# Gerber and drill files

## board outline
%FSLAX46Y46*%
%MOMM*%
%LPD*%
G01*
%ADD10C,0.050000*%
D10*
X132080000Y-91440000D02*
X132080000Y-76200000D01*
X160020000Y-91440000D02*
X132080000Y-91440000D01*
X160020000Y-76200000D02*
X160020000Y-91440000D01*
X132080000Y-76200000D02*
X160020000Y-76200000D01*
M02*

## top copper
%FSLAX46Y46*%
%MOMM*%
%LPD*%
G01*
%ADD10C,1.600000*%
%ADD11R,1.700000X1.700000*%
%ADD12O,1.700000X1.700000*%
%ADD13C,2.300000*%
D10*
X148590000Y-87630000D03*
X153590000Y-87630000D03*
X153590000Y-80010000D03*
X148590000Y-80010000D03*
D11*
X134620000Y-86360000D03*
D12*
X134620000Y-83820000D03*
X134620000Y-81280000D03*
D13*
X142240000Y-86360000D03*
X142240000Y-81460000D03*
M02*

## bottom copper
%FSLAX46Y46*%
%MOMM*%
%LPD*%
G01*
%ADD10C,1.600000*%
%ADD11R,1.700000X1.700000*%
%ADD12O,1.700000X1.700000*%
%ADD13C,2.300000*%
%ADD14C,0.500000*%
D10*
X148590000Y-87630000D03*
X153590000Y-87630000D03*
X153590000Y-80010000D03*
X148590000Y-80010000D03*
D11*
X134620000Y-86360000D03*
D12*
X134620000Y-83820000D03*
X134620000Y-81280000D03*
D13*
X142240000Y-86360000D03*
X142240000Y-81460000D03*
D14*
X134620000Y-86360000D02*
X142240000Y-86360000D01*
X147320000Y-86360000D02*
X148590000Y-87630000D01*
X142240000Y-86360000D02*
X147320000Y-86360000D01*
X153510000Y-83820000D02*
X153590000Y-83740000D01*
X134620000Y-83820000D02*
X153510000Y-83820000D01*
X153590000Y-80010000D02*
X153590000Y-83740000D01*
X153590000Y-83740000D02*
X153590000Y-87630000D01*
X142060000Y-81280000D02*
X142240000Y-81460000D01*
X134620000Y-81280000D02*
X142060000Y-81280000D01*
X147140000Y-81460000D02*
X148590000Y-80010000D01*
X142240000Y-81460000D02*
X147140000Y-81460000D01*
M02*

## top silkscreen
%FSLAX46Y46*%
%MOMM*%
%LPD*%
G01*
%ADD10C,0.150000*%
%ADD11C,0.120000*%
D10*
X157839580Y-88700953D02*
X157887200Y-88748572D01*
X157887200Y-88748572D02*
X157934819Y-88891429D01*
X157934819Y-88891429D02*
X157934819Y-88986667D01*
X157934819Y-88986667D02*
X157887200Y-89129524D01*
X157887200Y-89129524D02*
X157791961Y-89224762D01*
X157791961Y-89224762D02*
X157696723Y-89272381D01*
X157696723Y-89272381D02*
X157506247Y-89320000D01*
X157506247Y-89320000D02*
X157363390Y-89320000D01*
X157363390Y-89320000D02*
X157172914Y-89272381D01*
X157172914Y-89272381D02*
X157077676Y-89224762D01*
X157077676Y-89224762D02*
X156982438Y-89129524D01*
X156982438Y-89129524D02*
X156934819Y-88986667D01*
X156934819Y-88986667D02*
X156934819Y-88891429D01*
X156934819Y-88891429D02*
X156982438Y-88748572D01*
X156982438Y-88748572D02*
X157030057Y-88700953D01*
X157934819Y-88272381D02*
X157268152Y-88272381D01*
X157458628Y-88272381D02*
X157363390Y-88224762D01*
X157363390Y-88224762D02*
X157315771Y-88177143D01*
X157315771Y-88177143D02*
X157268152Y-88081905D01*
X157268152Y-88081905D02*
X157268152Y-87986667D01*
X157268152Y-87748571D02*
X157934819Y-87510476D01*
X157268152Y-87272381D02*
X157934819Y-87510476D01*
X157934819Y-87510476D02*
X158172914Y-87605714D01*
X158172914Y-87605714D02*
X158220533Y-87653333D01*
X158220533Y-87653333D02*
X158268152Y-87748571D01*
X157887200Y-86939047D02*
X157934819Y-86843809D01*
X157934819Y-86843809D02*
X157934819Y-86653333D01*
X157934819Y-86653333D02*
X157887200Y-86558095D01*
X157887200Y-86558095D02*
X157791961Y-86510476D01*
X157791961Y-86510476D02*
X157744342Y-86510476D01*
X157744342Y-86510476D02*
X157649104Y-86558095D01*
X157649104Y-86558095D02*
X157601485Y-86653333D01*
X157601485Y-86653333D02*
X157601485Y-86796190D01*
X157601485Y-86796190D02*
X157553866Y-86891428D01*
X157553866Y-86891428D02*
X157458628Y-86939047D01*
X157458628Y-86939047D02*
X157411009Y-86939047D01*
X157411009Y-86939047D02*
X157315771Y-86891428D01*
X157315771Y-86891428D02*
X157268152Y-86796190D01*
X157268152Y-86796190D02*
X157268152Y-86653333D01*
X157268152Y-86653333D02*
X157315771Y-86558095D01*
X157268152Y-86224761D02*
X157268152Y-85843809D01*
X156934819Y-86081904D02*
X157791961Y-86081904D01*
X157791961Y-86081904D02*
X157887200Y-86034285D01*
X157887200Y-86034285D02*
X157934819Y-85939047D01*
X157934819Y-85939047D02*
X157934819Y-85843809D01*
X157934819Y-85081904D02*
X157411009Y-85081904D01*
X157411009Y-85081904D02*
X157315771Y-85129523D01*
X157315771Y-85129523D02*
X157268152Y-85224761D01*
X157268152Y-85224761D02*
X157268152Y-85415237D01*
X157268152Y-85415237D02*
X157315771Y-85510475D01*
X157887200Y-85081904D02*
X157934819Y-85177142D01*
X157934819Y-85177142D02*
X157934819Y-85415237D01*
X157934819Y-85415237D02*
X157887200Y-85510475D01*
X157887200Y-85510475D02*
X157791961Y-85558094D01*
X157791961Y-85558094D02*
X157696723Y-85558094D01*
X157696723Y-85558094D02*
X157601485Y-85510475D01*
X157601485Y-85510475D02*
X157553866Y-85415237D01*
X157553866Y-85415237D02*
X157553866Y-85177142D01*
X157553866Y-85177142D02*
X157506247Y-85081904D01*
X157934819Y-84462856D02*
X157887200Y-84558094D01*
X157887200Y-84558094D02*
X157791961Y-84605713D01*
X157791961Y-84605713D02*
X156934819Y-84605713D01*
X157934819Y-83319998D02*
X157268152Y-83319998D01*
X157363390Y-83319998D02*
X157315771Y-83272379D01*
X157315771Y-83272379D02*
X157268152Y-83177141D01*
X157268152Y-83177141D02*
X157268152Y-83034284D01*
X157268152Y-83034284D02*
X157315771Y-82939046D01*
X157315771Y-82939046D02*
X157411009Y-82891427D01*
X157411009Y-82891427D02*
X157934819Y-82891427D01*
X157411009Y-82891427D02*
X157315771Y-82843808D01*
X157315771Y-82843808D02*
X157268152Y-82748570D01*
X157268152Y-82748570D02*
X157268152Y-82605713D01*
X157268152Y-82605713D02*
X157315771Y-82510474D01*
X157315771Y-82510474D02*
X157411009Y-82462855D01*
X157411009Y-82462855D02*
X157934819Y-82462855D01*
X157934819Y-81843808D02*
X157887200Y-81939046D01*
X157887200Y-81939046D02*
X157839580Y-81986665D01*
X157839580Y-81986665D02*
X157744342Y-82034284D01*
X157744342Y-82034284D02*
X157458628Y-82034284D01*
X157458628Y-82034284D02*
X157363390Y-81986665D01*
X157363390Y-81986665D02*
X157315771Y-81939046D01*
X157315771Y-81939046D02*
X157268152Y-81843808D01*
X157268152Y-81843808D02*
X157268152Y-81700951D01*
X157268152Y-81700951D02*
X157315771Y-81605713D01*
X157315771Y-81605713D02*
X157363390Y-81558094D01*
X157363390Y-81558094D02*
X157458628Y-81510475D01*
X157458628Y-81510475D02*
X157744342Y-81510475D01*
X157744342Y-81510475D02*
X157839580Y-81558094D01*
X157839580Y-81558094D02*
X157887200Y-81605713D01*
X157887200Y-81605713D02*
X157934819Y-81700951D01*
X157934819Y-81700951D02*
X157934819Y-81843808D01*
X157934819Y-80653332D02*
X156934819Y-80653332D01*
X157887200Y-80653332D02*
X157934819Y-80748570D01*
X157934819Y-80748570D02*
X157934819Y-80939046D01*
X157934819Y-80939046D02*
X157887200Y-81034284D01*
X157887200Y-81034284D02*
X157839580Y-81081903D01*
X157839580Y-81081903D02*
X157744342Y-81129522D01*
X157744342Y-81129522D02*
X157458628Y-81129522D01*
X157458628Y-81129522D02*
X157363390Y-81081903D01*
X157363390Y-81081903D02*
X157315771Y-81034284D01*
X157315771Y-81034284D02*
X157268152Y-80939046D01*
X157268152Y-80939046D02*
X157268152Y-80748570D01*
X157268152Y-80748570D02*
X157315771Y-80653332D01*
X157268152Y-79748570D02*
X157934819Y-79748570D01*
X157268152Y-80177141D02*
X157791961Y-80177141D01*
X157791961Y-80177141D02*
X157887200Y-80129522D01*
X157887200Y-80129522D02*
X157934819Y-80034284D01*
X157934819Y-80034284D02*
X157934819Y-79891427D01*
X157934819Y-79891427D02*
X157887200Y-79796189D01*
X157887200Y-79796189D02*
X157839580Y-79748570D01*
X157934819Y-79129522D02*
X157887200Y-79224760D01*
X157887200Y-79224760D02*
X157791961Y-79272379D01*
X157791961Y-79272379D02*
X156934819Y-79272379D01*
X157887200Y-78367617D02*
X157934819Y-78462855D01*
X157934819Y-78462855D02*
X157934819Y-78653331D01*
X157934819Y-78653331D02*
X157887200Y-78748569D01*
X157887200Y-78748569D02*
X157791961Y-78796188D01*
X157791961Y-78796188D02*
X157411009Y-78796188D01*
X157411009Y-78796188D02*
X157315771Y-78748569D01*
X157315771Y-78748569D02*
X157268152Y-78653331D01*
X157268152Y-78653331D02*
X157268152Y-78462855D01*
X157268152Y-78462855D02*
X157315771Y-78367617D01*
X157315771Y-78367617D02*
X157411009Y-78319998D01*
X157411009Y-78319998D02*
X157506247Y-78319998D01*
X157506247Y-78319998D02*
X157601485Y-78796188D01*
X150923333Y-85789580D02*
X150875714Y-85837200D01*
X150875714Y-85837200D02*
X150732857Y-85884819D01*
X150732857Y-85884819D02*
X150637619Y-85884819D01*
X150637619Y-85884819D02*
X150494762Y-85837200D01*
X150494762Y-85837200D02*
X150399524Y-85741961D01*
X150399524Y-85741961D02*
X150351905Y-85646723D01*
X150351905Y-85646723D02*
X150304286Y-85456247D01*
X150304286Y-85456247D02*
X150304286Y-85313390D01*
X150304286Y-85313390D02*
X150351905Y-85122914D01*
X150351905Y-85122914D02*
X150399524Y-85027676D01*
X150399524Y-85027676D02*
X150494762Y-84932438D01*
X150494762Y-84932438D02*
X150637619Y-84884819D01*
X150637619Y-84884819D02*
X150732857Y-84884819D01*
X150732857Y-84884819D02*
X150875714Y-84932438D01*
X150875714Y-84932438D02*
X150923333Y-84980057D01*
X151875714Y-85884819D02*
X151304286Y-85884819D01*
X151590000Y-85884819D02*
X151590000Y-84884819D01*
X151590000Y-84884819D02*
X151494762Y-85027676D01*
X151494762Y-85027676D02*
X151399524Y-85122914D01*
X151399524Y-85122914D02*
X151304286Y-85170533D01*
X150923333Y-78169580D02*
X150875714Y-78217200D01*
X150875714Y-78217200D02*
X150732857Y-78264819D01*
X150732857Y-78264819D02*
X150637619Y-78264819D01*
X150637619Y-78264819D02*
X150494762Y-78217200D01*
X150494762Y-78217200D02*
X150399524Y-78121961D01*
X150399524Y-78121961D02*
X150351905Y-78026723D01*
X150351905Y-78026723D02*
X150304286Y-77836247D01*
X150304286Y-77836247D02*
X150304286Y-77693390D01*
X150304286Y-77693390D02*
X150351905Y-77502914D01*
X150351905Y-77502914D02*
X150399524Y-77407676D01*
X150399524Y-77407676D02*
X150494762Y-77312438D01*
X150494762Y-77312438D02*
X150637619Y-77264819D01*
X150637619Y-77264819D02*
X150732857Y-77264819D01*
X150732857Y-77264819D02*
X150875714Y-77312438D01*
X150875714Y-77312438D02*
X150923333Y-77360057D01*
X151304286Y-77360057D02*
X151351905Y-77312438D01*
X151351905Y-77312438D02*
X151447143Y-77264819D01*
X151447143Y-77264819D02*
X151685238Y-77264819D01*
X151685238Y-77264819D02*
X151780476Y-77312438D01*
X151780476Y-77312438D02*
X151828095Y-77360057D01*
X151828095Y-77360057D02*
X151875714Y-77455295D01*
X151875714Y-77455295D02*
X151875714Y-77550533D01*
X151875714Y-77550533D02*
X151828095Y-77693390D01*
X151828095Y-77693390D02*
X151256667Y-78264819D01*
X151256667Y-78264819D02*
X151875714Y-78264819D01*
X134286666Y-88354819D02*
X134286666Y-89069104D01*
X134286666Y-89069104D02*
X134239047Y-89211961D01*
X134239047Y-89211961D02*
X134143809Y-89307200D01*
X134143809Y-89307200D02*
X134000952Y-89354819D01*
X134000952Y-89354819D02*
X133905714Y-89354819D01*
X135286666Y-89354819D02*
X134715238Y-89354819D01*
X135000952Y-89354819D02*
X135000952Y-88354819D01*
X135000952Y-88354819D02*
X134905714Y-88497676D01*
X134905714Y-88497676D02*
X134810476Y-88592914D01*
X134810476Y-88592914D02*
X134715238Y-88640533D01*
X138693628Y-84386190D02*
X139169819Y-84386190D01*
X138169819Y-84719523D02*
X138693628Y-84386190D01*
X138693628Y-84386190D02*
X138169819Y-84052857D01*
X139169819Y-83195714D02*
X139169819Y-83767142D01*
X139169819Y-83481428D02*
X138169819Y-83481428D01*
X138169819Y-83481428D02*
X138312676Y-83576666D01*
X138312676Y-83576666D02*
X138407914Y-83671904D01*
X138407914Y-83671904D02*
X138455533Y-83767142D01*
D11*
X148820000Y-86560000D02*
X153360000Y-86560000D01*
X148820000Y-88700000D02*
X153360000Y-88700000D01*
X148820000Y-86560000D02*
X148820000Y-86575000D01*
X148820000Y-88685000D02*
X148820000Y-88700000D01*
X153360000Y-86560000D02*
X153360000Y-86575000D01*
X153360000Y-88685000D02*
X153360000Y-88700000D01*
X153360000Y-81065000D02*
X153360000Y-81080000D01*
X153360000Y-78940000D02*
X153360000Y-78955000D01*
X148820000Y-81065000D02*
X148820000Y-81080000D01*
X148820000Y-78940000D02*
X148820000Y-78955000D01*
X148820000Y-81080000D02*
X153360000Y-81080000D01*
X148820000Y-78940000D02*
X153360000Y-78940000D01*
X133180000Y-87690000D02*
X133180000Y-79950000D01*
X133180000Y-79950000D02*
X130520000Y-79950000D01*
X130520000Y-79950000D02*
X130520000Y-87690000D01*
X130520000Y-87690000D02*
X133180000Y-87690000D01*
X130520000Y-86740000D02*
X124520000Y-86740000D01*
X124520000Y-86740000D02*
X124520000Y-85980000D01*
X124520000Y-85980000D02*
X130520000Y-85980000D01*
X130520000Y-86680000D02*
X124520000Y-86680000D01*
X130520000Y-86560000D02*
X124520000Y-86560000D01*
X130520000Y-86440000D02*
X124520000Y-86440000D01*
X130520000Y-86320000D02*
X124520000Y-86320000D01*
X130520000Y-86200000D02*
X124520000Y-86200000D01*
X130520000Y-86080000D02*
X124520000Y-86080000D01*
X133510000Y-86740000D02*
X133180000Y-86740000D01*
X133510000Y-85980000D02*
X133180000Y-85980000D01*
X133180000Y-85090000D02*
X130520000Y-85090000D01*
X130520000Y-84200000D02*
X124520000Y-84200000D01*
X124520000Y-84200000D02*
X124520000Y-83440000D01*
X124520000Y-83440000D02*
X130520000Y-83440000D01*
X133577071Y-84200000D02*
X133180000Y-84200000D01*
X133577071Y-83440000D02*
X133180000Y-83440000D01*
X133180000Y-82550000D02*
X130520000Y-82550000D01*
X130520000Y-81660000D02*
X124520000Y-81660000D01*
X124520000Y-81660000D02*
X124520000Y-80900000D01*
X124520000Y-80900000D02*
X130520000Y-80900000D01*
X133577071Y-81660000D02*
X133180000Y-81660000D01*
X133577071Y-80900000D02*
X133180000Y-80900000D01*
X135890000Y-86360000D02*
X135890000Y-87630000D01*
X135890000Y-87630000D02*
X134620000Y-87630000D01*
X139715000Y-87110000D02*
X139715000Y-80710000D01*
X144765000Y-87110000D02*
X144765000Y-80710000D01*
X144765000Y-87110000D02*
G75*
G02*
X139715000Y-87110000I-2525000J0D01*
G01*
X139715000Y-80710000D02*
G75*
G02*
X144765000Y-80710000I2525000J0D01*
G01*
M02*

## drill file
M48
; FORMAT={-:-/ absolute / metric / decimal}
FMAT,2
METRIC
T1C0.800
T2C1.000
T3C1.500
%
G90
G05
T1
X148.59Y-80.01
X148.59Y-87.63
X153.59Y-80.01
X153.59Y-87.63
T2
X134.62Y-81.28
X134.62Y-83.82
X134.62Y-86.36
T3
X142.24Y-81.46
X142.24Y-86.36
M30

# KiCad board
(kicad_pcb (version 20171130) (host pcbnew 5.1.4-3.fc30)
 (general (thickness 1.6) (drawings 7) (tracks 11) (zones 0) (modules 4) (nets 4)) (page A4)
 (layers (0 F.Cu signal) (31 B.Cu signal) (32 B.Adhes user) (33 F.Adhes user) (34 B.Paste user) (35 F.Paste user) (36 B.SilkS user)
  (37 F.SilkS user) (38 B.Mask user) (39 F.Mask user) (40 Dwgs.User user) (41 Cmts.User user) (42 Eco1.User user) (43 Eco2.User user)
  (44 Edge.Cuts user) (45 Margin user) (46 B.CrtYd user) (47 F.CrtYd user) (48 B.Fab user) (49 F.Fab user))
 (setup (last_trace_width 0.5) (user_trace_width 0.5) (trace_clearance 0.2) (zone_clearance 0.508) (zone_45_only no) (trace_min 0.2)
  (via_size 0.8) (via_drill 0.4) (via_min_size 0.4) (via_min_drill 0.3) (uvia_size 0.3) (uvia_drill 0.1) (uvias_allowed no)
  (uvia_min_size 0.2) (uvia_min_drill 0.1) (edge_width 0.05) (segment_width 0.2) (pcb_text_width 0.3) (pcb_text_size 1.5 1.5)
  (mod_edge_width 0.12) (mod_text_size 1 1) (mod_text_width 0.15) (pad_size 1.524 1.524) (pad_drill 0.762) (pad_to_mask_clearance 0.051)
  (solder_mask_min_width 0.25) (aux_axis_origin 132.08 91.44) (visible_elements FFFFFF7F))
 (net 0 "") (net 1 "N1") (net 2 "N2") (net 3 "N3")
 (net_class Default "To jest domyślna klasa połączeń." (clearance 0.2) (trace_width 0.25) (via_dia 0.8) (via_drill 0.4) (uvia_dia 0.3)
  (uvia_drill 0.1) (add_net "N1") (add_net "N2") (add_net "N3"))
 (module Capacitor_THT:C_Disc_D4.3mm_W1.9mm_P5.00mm (layer F.Cu) (at 148.59 87.63)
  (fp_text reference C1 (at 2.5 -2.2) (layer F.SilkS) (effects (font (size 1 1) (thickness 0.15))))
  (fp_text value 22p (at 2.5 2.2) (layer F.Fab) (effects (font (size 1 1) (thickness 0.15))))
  (fp_line (start 0.23 -1.07) (end 4.77 -1.07) (layer F.SilkS) (width 0.12))
  (fp_line (start 0.23 1.07) (end 4.77 1.07) (layer F.SilkS) (width 0.12))
  (fp_line (start 0.23 -1.07) (end 0.23 -1.055) (layer F.SilkS) (width 0.12))
  (fp_line (start 0.23 1.055) (end 0.23 1.07) (layer F.SilkS) (width 0.12))
  (fp_line (start 4.77 -1.07) (end 4.77 -1.055) (layer F.SilkS) (width 0.12))
  (fp_line (start 4.77 1.055) (end 4.77 1.07) (layer F.SilkS) (width 0.12))
  (pad 1 thru_hole circle (at 0 0) (size 1.6 1.6) (drill 0.8) (layers *.Cu *.Mask) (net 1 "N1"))
  (pad 2 thru_hole circle (at 5 0) (size 1.6 1.6) (drill 0.8) (layers *.Cu *.Mask) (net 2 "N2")))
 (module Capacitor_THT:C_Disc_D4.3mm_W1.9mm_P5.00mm (layer F.Cu) (at 148.59 80.01)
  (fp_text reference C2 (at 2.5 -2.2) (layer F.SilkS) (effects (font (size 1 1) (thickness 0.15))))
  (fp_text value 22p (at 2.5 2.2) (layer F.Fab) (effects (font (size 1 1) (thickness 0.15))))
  (fp_line (start 4.77 1.055) (end 4.77 1.07) (layer F.SilkS) (width 0.12))
  (fp_line (start 4.77 -1.07) (end 4.77 -1.055) (layer F.SilkS) (width 0.12))
  (fp_line (start 0.23 1.055) (end 0.23 1.07) (layer F.SilkS) (width 0.12))
  (fp_line (start 0.23 -1.07) (end 0.23 -1.055) (layer F.SilkS) (width 0.12))
  (fp_line (start 0.23 1.07) (end 4.77 1.07) (layer F.SilkS) (width 0.12))
  (fp_line (start 0.23 -1.07) (end 4.77 -1.07) (layer F.SilkS) (width 0.12))
  (pad 2 thru_hole circle (at 5 0) (size 1.6 1.6) (drill 0.8) (layers *.Cu *.Mask) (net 2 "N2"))
  (pad 1 thru_hole circle (at 0 0) (size 1.6 1.6) (drill 0.8) (layers *.Cu *.Mask) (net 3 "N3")))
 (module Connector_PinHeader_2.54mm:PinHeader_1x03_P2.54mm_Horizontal (layer F.Cu) (at 134.62 86.36 180)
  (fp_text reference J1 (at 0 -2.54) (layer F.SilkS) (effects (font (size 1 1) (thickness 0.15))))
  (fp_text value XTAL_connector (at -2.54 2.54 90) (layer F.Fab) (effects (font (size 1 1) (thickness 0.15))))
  (fp_line (start 1.44 -1.33) (end 1.44 6.41) (layer F.SilkS) (width 0.12))
  (fp_line (start 1.44 6.41) (end 4.1 6.41) (layer F.SilkS) (width 0.12))
  (fp_line (start 4.1 6.41) (end 4.1 -1.33) (layer F.SilkS) (width 0.12))
  (fp_line (start 4.1 -1.33) (end 1.44 -1.33) (layer F.SilkS) (width 0.12))
  (fp_line (start 4.1 -0.38) (end 10.1 -0.38) (layer F.SilkS) (width 0.12))
  (fp_line (start 10.1 -0.38) (end 10.1 0.38) (layer F.SilkS) (width 0.12))
  (fp_line (start 10.1 0.38) (end 4.1 0.38) (layer F.SilkS) (width 0.12))
  (fp_line (start 4.1 -0.32) (end 10.1 -0.32) (layer F.SilkS) (width 0.12))
  (fp_line (start 4.1 -0.2) (end 10.1 -0.2) (layer F.SilkS) (width 0.12))
  (fp_line (start 4.1 -0.08) (end 10.1 -0.08) (layer F.SilkS) (width 0.12))
  (fp_line (start 4.1 0.04) (end 10.1 0.04) (layer F.SilkS) (width 0.12))
  (fp_line (start 4.1 0.16) (end 10.1 0.16) (layer F.SilkS) (width 0.12))
  (fp_line (start 4.1 0.28) (end 10.1 0.28) (layer F.SilkS) (width 0.12))
  (fp_line (start 1.11 -0.38) (end 1.44 -0.38) (layer F.SilkS) (width 0.12))
  (fp_line (start 1.11 0.38) (end 1.44 0.38) (layer F.SilkS) (width 0.12))
  (fp_line (start 1.44 1.27) (end 4.1 1.27) (layer F.SilkS) (width 0.12))
  (fp_line (start 4.1 2.16) (end 10.1 2.16) (layer F.SilkS) (width 0.12))
  (fp_line (start 10.1 2.16) (end 10.1 2.92) (layer F.SilkS) (width 0.12))
  (fp_line (start 10.1 2.92) (end 4.1 2.92) (layer F.SilkS) (width 0.12))
  (fp_line (start 1.042929 2.16) (end 1.44 2.16) (layer F.SilkS) (width 0.12))
  (fp_line (start 1.042929 2.92) (end 1.44 2.92) (layer F.SilkS) (width 0.12))
  (fp_line (start 1.44 3.81) (end 4.1 3.81) (layer F.SilkS) (width 0.12))
  (fp_line (start 4.1 4.7) (end 10.1 4.7) (layer F.SilkS) (width 0.12))
  (fp_line (start 10.1 4.7) (end 10.1 5.46) (layer F.SilkS) (width 0.12))
  (fp_line (start 10.1 5.46) (end 4.1 5.46) (layer F.SilkS) (width 0.12))
  (fp_line (start 1.042929 4.7) (end 1.44 4.7) (layer F.SilkS) (width 0.12))
  (fp_line (start 1.042929 5.46) (end 1.44 5.46) (layer F.SilkS) (width 0.12))
  (fp_line (start -1.27 0) (end -1.27 -1.27) (layer F.SilkS) (width 0.12))
  (fp_line (start -1.27 -1.27) (end 0 -1.27) (layer F.SilkS) (width 0.12))
  (pad 1 thru_hole rect (at 0 0 180) (size 1.7 1.7) (drill 1) (layers *.Cu *.Mask) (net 1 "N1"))
  (pad 2 thru_hole oval (at 0 2.54 180) (size 1.7 1.7) (drill 1) (layers *.Cu *.Mask) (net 2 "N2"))
  (pad 3 thru_hole oval (at 0 5.08 180) (size 1.7 1.7) (drill 1) (layers *.Cu *.Mask) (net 3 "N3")))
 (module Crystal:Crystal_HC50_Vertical (layer F.Cu) (at 142.24 86.36 90)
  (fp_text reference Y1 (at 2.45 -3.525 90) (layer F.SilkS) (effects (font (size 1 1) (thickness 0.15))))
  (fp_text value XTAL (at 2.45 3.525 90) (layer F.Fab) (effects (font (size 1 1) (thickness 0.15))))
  (fp_line (start -0.75 -2.525) (end 5.65 -2.525) (layer F.SilkS) (width 0.12))
  (fp_line (start -0.75 2.525) (end 5.65 2.525) (layer F.SilkS) (width 0.12))
  (fp_arc (start -0.75 0) (end -0.75 -2.525) (angle -180) (layer F.SilkS) (width 0.12))
  (fp_arc (start 5.65 0) (end 5.65 -2.525) (angle 180) (layer F.SilkS) (width 0.12))
  (pad 1 thru_hole circle (at 0 0 90) (size 2.3 2.3) (drill 1.5) (layers *.Cu *.Mask) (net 1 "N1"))
  (pad 2 thru_hole circle (at 4.9 0 90) (size 2.3 2.3) (drill 1.5) (layers *.Cu *.Mask) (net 3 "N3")))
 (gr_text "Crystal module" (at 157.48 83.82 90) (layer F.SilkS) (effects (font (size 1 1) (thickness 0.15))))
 (gr_line (start 132.08 91.44) (end 132.08 76.2) (layer Edge.Cuts) (width 0.05))
 (gr_line (start 160.02 91.44) (end 132.08 91.44) (layer Edge.Cuts) (width 0.05))
 (gr_line (start 160.02 76.2) (end 160.02 91.44) (layer Edge.Cuts) (width 0.05))
 (gr_line (start 132.08 76.2) (end 160.02 76.2) (layer Edge.Cuts) (width 0.05))
 (segment (start 134.62 86.36) (end 142.24 86.36) (width 0.5) (layer B.Cu) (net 1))
 (segment (start 147.32 86.36) (end 148.59 87.63) (width 0.5) (layer B.Cu) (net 1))
 (segment (start 142.24 86.36) (end 147.32 86.36) (width 0.5) (layer B.Cu) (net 1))
 (segment (start 153.51 83.82) (end 153.59 83.74) (width 0.5) (layer B.Cu) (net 2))
 (segment (start 134.62 83.82) (end 153.51 83.82) (width 0.5) (layer B.Cu) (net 2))
 (segment (start 153.59 80.01) (end 153.59 83.74) (width 0.5) (layer B.Cu) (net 2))
 (segment (start 153.59 83.74) (end 153.59 87.63) (width 0.5) (layer B.Cu) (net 2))
 (segment (start 142.06 81.28) (end 142.24 81.46) (width 0.5) (layer B.Cu) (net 3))
 (segment (start 134.62 81.28) (end 142.06 81.28) (width 0.5) (layer B.Cu) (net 3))
 (segment (start 147.14 81.46) (end 148.59 80.01) (width 0.5) (layer B.Cu) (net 3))
 (segment (start 142.24 81.46) (end 147.14 81.46) (width 0.5) (layer B.Cu) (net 3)))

